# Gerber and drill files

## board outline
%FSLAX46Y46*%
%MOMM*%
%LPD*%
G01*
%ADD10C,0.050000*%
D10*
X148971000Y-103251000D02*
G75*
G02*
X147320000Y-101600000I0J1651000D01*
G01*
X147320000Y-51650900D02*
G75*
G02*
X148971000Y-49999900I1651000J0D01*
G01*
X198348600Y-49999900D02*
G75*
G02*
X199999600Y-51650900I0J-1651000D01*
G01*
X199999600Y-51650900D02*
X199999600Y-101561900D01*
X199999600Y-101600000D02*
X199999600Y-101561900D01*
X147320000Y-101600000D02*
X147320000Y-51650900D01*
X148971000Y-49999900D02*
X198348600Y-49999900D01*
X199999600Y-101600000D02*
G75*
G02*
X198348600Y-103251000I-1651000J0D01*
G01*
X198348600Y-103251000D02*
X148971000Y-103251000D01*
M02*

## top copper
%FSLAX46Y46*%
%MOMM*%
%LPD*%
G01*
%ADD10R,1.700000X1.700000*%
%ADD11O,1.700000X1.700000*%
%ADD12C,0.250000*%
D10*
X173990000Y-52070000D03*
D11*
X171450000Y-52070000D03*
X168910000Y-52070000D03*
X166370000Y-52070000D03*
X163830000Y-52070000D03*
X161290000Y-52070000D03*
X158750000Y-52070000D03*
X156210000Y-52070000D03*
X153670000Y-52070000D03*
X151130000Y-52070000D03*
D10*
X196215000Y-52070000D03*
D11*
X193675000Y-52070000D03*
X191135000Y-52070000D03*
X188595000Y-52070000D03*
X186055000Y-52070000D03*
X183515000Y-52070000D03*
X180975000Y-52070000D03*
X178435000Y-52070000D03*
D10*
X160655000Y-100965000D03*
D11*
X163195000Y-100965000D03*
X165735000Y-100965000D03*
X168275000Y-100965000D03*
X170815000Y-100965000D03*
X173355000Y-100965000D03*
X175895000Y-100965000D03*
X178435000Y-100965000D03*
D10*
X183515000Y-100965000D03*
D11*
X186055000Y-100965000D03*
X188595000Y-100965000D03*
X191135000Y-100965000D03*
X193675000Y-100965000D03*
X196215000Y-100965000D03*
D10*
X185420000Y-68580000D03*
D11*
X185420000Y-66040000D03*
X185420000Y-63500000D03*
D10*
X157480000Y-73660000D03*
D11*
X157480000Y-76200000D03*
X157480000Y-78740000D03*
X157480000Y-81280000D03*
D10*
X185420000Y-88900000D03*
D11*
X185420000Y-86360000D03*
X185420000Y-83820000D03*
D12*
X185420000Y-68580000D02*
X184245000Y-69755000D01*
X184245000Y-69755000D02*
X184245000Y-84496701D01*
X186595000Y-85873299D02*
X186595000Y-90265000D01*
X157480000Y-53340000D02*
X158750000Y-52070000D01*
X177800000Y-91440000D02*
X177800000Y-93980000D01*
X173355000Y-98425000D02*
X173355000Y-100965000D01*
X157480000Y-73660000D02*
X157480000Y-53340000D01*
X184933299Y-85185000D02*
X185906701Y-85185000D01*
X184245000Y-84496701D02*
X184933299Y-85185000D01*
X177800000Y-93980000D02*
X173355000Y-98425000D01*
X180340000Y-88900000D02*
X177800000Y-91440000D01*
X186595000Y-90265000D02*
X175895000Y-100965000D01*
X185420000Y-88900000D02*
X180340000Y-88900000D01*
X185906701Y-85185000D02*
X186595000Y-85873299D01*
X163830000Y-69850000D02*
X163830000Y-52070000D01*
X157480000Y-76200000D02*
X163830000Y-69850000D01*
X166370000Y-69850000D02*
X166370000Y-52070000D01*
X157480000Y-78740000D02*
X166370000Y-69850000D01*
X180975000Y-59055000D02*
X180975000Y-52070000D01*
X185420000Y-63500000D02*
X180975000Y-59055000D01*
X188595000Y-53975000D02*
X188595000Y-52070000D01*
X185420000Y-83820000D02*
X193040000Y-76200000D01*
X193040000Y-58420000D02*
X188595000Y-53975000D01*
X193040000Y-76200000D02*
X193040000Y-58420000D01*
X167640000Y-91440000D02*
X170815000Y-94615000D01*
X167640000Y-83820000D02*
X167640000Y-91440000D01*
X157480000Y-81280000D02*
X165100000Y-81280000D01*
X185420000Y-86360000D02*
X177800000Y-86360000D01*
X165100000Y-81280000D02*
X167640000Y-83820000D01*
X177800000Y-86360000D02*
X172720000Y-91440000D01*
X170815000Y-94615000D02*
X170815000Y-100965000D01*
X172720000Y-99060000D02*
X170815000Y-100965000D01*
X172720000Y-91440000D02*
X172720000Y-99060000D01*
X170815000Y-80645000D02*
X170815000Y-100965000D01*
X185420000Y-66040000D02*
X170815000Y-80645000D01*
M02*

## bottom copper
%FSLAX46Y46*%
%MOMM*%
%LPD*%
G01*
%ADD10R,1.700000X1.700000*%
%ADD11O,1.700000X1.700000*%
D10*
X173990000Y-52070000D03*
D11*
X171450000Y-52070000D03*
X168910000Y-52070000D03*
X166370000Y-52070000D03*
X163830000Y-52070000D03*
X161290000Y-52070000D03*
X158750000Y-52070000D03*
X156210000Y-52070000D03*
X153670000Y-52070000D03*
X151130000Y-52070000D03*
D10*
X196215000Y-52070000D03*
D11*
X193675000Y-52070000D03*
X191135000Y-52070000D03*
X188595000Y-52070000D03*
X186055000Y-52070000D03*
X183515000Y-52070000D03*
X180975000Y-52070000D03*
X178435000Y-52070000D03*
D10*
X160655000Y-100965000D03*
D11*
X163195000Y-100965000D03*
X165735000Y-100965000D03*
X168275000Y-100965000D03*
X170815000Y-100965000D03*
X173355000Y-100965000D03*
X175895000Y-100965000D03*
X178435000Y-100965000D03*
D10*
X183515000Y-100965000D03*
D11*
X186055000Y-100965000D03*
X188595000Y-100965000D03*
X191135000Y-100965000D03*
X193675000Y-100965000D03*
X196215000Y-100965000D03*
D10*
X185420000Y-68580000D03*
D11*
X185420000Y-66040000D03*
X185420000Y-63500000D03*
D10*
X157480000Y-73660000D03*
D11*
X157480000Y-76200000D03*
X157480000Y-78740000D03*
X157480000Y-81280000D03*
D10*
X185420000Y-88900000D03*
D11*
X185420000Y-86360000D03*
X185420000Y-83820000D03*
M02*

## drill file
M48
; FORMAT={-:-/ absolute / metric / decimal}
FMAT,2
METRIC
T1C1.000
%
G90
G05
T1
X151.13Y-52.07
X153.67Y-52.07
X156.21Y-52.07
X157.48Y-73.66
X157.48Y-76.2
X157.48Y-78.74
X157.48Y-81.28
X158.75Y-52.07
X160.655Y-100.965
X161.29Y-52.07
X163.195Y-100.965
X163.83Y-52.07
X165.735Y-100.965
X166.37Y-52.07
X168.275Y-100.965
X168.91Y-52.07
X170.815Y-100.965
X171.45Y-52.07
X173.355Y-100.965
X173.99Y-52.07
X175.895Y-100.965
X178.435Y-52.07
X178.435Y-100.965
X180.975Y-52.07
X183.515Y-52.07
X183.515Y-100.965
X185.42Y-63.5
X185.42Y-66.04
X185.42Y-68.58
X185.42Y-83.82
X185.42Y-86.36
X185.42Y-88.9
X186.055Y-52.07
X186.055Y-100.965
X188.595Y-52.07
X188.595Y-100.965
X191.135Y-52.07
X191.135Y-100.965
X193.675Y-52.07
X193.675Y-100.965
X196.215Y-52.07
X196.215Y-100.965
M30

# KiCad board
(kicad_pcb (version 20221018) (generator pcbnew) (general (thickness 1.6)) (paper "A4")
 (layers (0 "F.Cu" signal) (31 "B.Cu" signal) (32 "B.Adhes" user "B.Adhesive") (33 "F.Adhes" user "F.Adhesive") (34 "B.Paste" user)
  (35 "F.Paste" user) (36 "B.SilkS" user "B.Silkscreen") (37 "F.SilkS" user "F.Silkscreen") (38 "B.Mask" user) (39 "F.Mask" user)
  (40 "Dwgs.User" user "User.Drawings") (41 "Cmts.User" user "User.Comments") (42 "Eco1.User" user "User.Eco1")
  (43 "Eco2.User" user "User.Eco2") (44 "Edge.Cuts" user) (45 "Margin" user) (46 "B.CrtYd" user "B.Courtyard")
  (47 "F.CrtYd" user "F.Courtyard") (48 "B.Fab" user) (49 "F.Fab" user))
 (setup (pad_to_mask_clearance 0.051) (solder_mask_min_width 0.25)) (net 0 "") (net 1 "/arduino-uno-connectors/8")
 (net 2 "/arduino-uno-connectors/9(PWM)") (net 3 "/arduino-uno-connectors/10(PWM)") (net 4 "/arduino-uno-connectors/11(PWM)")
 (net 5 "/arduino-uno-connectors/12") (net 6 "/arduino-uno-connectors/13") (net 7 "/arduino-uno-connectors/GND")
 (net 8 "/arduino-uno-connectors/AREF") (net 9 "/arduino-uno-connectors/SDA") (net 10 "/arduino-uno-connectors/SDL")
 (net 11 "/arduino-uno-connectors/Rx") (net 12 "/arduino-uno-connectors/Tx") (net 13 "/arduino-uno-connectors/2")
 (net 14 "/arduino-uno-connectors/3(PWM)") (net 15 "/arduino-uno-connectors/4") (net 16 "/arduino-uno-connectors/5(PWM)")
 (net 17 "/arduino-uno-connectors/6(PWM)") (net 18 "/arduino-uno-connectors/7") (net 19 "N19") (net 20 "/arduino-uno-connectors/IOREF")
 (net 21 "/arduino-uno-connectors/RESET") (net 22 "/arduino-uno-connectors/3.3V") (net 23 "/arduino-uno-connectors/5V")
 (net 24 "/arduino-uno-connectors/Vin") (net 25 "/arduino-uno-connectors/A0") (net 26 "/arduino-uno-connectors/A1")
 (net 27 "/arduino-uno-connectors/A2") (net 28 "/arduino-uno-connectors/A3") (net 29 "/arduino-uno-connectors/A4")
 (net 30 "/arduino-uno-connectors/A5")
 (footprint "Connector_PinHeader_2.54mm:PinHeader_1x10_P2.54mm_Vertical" (layer "F.Cu") (at 173.99 52.07 -90)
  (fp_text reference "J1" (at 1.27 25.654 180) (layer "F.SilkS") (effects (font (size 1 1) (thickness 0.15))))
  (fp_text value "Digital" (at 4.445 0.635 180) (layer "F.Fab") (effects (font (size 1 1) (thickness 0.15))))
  (pad "1" thru_hole rect (at 0 0 270) (size 1.7 1.7) (drill 1) (layers "*.Cu" "*.Mask") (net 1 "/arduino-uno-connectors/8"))
  (pad "2" thru_hole oval (at 0 2.54 270) (size 1.7 1.7) (drill 1) (layers "*.Cu" "*.Mask") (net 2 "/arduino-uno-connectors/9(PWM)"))
  (pad "3" thru_hole oval (at 0 5.08 270) (size 1.7 1.7) (drill 1) (layers "*.Cu" "*.Mask") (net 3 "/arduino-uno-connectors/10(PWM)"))
  (pad "4" thru_hole oval (at 0 7.62 270) (size 1.7 1.7) (drill 1) (layers "*.Cu" "*.Mask") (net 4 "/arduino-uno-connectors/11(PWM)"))
  (pad "5" thru_hole oval (at 0 10.16 270) (size 1.7 1.7) (drill 1) (layers "*.Cu" "*.Mask") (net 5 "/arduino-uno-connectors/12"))
  (pad "6" thru_hole oval (at 0 12.7 270) (size 1.7 1.7) (drill 1) (layers "*.Cu" "*.Mask") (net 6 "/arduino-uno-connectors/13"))
  (pad "7" thru_hole oval (at 0 15.24 270) (size 1.7 1.7) (drill 1) (layers "*.Cu" "*.Mask") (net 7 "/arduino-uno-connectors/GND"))
  (pad "8" thru_hole oval (at 0 17.78 270) (size 1.7 1.7) (drill 1) (layers "*.Cu" "*.Mask") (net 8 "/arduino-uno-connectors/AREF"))
  (pad "9" thru_hole oval (at 0 20.32 270) (size 1.7 1.7) (drill 1) (layers "*.Cu" "*.Mask") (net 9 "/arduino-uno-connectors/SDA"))
  (pad "10" thru_hole oval (at 0 22.86 270) (size 1.7 1.7) (drill 1) (layers "*.Cu" "*.Mask") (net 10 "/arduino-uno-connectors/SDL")))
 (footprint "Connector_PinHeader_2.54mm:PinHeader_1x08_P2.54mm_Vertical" (layer "F.Cu") (at 196.215 52.07 -90)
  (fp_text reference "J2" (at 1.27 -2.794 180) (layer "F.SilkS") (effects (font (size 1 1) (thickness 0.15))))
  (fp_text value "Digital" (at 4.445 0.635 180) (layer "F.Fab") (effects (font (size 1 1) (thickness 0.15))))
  (pad "1" thru_hole rect (at 0 0 270) (size 1.7 1.7) (drill 1) (layers "*.Cu" "*.Mask") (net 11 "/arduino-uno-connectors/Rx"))
  (pad "2" thru_hole oval (at 0 2.54 270) (size 1.7 1.7) (drill 1) (layers "*.Cu" "*.Mask") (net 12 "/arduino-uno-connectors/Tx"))
  (pad "3" thru_hole oval (at 0 5.08 270) (size 1.7 1.7) (drill 1) (layers "*.Cu" "*.Mask") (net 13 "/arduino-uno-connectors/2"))
  (pad "4" thru_hole oval (at 0 7.62 270) (size 1.7 1.7) (drill 1) (layers "*.Cu" "*.Mask") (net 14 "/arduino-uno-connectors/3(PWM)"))
  (pad "5" thru_hole oval (at 0 10.16 270) (size 1.7 1.7) (drill 1) (layers "*.Cu" "*.Mask") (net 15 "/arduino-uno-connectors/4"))
  (pad "6" thru_hole oval (at 0 12.7 270) (size 1.7 1.7) (drill 1) (layers "*.Cu" "*.Mask") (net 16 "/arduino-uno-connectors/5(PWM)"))
  (pad "7" thru_hole oval (at 0 15.24 270) (size 1.7 1.7) (drill 1) (layers "*.Cu" "*.Mask") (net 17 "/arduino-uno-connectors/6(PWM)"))
  (pad "8" thru_hole oval (at 0 17.78 270) (size 1.7 1.7) (drill 1) (layers "*.Cu" "*.Mask") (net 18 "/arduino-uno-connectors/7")))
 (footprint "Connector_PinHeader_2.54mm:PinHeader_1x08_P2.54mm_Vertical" (layer "F.Cu") (at 160.655 100.965 90)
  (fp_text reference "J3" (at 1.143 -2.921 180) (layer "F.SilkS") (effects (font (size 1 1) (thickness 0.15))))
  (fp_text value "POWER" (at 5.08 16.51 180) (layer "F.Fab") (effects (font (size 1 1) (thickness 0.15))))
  (pad "1" thru_hole rect (at 0 0 90) (size 1.7 1.7) (drill 1) (layers "*.Cu" "*.Mask") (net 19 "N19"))
  (pad "2" thru_hole oval (at 0 2.54 90) (size 1.7 1.7) (drill 1) (layers "*.Cu" "*.Mask") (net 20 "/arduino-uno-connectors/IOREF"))
  (pad "3" thru_hole oval (at 0 5.08 90) (size 1.7 1.7) (drill 1) (layers "*.Cu" "*.Mask") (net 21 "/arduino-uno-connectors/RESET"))
  (pad "4" thru_hole oval (at 0 7.62 90) (size 1.7 1.7) (drill 1) (layers "*.Cu" "*.Mask") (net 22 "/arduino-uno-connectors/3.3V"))
  (pad "5" thru_hole oval (at 0 10.16 90) (size 1.7 1.7) (drill 1) (layers "*.Cu" "*.Mask") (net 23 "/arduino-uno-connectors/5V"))
  (pad "6" thru_hole oval (at 0 12.7 90) (size 1.7 1.7) (drill 1) (layers "*.Cu" "*.Mask") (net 7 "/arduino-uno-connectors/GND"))
  (pad "7" thru_hole oval (at 0 15.24 90) (size 1.7 1.7) (drill 1) (layers "*.Cu" "*.Mask") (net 7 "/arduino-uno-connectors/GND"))
  (pad "8" thru_hole oval (at 0 17.78 90) (size 1.7 1.7) (drill 1) (layers "*.Cu" "*.Mask") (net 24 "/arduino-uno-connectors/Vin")))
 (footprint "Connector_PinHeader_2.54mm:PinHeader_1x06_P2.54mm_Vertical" (layer "F.Cu") (at 183.515 100.965 90)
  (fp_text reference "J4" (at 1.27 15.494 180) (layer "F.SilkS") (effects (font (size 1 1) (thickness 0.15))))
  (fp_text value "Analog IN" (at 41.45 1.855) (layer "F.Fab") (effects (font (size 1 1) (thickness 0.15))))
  (pad "1" thru_hole rect (at 0 0 90) (size 1.7 1.7) (drill 1) (layers "*.Cu" "*.Mask") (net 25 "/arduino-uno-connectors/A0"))
  (pad "2" thru_hole oval (at 0 2.54 90) (size 1.7 1.7) (drill 1) (layers "*.Cu" "*.Mask") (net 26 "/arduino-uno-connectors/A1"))
  (pad "3" thru_hole oval (at 0 5.08 90) (size 1.7 1.7) (drill 1) (layers "*.Cu" "*.Mask") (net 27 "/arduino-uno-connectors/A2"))
  (pad "4" thru_hole oval (at 0 7.62 90) (size 1.7 1.7) (drill 1) (layers "*.Cu" "*.Mask") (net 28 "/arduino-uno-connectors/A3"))
  (pad "5" thru_hole oval (at 0 10.16 90) (size 1.7 1.7) (drill 1) (layers "*.Cu" "*.Mask") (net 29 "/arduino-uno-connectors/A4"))
  (pad "6" thru_hole oval (at 0 12.7 90) (size 1.7 1.7) (drill 1) (layers "*.Cu" "*.Mask") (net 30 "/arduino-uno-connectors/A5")))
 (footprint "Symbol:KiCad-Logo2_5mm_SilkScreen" (layer "F.Cu") (at 153.8478 60.0964)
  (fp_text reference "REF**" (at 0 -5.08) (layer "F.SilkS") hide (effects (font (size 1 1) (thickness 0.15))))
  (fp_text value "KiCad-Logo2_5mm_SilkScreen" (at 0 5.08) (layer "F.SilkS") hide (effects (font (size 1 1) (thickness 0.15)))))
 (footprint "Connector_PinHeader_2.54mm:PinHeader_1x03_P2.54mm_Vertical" (layer "F.Cu") (at 185.42 68.58 180)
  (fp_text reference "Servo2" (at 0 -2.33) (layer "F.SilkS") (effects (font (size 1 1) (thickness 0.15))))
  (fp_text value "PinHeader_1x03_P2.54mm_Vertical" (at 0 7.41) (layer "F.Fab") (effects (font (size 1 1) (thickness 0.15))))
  (pad "1" thru_hole rect (at 0 0 180) (size 1.7 1.7) (drill 1) (layers "*.Cu" "*.Mask") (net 7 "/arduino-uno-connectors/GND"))
  (pad "2" thru_hole oval (at 0 2.54 180) (size 1.7 1.7) (drill 1) (layers "*.Cu" "*.Mask") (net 23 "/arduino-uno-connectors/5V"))
  (pad "3" thru_hole oval (at 0 5.08 180) (size 1.7 1.7) (drill 1) (layers "*.Cu" "*.Mask") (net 17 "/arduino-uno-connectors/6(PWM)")))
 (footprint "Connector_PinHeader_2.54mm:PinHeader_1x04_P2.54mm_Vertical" (layer "F.Cu") (at 157.48 73.66)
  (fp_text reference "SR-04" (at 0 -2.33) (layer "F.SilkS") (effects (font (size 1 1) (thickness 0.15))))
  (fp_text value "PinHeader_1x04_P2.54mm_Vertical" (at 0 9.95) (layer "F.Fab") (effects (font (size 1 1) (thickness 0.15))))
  (pad "1" thru_hole rect (at 0 0) (size 1.7 1.7) (drill 1) (layers "*.Cu" "*.Mask") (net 7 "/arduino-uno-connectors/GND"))
  (pad "2" thru_hole oval (at 0 2.54) (size 1.7 1.7) (drill 1) (layers "*.Cu" "*.Mask") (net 5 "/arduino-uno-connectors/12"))
  (pad "3" thru_hole oval (at 0 5.08) (size 1.7 1.7) (drill 1) (layers "*.Cu" "*.Mask") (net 4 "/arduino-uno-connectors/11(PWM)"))
  (pad "4" thru_hole oval (at 0 7.62) (size 1.7 1.7) (drill 1) (layers "*.Cu" "*.Mask") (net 23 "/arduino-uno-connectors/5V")))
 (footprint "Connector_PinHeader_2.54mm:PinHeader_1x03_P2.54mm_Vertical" (layer "F.Cu") (at 185.42 88.9 180)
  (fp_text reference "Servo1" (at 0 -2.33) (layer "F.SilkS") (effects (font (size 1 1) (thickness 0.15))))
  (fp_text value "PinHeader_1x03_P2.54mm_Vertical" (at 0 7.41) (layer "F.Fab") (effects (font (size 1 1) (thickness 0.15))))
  (pad "1" thru_hole rect (at 0 0 180) (size 1.7 1.7) (drill 1) (layers "*.Cu" "*.Mask") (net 7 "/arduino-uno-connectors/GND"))
  (pad "2" thru_hole oval (at 0 2.54 180) (size 1.7 1.7) (drill 1) (layers "*.Cu" "*.Mask") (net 23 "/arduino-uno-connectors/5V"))
  (pad "3" thru_hole oval (at 0 5.08 180) (size 1.7 1.7) (drill 1) (layers "*.Cu" "*.Mask") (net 14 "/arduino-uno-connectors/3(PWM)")))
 (gr_arc (start 148.971 103.251) (mid 147.803567 102.767433) (end 147.32 101.6) (stroke (width 0.05) (type solid)) (layer "Edge.Cuts"))
 (gr_arc (start 147.32 51.6509) (mid 147.803567 50.483467) (end 148.971 49.9999) (stroke (width 0.05) (type solid)) (layer "Edge.Cuts"))
 (gr_arc (start 198.3486 49.9999) (mid 199.516033 50.483467) (end 199.9996 51.6509) (stroke (width 0.05) (type solid)) (layer "Edge.Cuts"))
 (gr_line (start 199.9996 51.6509) (end 199.9996 101.5619) (stroke (width 0.05) (type solid)) (layer "Edge.Cuts"))
 (gr_line (start 199.9996 101.6) (end 199.9996 101.5619) (stroke (width 0.05) (type solid)) (layer "Edge.Cuts"))
 (gr_line (start 147.32 101.6) (end 147.32 51.6509) (stroke (width 0.05) (type solid)) (layer "Edge.Cuts"))
 (gr_line (start 148.971 49.9999) (end 198.3486 49.9999) (stroke (width 0.05) (type solid)) (layer "Edge.Cuts"))
 (gr_arc (start 199.9996 101.6) (mid 199.516033 102.767433) (end 198.3486 103.251) (stroke (width 0.05) (type solid)) (layer "Edge.Cuts"))
 (gr_line (start 198.3486 103.251) (end 148.971 103.251) (stroke (width 0.05) (type solid)) (layer "Edge.Cuts"))
 (segment (start 185.42 68.58) (end 184.245 69.755) (width 0.25) (layer "F.Cu") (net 7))
 (segment (start 184.245 69.755) (end 184.245 84.496701) (width 0.25) (layer "F.Cu") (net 7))
 (segment (start 186.595 85.873299) (end 186.595 90.265) (width 0.25) (layer "F.Cu") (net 7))
 (segment (start 157.48 53.34) (end 158.75 52.07) (width 0.25) (layer "F.Cu") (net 7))
 (segment (start 177.8 91.44) (end 177.8 93.98) (width 0.25) (layer "F.Cu") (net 7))
 (segment (start 173.355 98.425) (end 173.355 100.965) (width 0.25) (layer "F.Cu") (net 7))
 (segment (start 157.48 73.66) (end 157.48 53.34) (width 0.25) (layer "F.Cu") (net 7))
 (segment (start 184.933299 85.185) (end 185.906701 85.185) (width 0.25) (layer "F.Cu") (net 7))
 (segment (start 184.245 84.496701) (end 184.933299 85.185) (width 0.25) (layer "F.Cu") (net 7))
 (segment (start 177.8 93.98) (end 173.355 98.425) (width 0.25) (layer "F.Cu") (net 7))
 (segment (start 180.34 88.9) (end 177.8 91.44) (width 0.25) (layer "F.Cu") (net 7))
 (segment (start 186.595 90.265) (end 175.895 100.965) (width 0.25) (layer "F.Cu") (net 7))
 (segment (start 185.42 88.9) (end 180.34 88.9) (width 0.25) (layer "F.Cu") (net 7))
 (segment (start 185.906701 85.185) (end 186.595 85.873299) (width 0.25) (layer "F.Cu") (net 7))
 (segment (start 163.83 69.85) (end 163.83 52.07) (width 0.25) (layer "F.Cu") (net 5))
 (segment (start 157.48 76.2) (end 163.83 69.85) (width 0.25) (layer "F.Cu") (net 5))
 (segment (start 166.37 69.85) (end 166.37 52.07) (width 0.25) (layer "F.Cu") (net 4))
 (segment (start 157.48 78.74) (end 166.37 69.85) (width 0.25) (layer "F.Cu") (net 4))
 (segment (start 180.975 59.055) (end 180.975 52.07) (width 0.25) (layer "F.Cu") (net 17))
 (segment (start 185.42 63.5) (end 180.975 59.055) (width 0.25) (layer "F.Cu") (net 17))
 (segment (start 188.595 53.975) (end 188.595 52.07) (width 0.25) (layer "F.Cu") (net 14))
 (segment (start 185.42 83.82) (end 193.04 76.2) (width 0.25) (layer "F.Cu") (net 14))
 (segment (start 193.04 58.42) (end 188.595 53.975) (width 0.25) (layer "F.Cu") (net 14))
 (segment (start 193.04 76.2) (end 193.04 58.42) (width 0.25) (layer "F.Cu") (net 14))
 (segment (start 167.64 91.44) (end 170.815 94.615) (width 0.25) (layer "F.Cu") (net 23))
 (segment (start 167.64 83.82) (end 167.64 91.44) (width 0.25) (layer "F.Cu") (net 23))
 (segment (start 157.48 81.28) (end 165.1 81.28) (width 0.25) (layer "F.Cu") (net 23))
 (segment (start 185.42 86.36) (end 177.8 86.36) (width 0.25) (layer "F.Cu") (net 23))
 (segment (start 165.1 81.28) (end 167.64 83.82) (width 0.25) (layer "F.Cu") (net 23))
 (segment (start 177.8 86.36) (end 172.72 91.44) (width 0.25) (layer "F.Cu") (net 23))
 (segment (start 170.815 94.615) (end 170.815 100.965) (width 0.25) (layer "F.Cu") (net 23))
 (segment (start 172.72 99.06) (end 170.815 100.965) (width 0.25) (layer "F.Cu") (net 23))
 (segment (start 172.72 91.44) (end 172.72 99.06) (width 0.25) (layer "F.Cu") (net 23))
 (segment (start 170.815 80.645) (end 170.815 100.965) (width 0.25) (layer "F.Cu") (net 23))
 (segment (start 185.42 66.04) (end 170.815 80.645) (width 0.25) (layer "F.Cu") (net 23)))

